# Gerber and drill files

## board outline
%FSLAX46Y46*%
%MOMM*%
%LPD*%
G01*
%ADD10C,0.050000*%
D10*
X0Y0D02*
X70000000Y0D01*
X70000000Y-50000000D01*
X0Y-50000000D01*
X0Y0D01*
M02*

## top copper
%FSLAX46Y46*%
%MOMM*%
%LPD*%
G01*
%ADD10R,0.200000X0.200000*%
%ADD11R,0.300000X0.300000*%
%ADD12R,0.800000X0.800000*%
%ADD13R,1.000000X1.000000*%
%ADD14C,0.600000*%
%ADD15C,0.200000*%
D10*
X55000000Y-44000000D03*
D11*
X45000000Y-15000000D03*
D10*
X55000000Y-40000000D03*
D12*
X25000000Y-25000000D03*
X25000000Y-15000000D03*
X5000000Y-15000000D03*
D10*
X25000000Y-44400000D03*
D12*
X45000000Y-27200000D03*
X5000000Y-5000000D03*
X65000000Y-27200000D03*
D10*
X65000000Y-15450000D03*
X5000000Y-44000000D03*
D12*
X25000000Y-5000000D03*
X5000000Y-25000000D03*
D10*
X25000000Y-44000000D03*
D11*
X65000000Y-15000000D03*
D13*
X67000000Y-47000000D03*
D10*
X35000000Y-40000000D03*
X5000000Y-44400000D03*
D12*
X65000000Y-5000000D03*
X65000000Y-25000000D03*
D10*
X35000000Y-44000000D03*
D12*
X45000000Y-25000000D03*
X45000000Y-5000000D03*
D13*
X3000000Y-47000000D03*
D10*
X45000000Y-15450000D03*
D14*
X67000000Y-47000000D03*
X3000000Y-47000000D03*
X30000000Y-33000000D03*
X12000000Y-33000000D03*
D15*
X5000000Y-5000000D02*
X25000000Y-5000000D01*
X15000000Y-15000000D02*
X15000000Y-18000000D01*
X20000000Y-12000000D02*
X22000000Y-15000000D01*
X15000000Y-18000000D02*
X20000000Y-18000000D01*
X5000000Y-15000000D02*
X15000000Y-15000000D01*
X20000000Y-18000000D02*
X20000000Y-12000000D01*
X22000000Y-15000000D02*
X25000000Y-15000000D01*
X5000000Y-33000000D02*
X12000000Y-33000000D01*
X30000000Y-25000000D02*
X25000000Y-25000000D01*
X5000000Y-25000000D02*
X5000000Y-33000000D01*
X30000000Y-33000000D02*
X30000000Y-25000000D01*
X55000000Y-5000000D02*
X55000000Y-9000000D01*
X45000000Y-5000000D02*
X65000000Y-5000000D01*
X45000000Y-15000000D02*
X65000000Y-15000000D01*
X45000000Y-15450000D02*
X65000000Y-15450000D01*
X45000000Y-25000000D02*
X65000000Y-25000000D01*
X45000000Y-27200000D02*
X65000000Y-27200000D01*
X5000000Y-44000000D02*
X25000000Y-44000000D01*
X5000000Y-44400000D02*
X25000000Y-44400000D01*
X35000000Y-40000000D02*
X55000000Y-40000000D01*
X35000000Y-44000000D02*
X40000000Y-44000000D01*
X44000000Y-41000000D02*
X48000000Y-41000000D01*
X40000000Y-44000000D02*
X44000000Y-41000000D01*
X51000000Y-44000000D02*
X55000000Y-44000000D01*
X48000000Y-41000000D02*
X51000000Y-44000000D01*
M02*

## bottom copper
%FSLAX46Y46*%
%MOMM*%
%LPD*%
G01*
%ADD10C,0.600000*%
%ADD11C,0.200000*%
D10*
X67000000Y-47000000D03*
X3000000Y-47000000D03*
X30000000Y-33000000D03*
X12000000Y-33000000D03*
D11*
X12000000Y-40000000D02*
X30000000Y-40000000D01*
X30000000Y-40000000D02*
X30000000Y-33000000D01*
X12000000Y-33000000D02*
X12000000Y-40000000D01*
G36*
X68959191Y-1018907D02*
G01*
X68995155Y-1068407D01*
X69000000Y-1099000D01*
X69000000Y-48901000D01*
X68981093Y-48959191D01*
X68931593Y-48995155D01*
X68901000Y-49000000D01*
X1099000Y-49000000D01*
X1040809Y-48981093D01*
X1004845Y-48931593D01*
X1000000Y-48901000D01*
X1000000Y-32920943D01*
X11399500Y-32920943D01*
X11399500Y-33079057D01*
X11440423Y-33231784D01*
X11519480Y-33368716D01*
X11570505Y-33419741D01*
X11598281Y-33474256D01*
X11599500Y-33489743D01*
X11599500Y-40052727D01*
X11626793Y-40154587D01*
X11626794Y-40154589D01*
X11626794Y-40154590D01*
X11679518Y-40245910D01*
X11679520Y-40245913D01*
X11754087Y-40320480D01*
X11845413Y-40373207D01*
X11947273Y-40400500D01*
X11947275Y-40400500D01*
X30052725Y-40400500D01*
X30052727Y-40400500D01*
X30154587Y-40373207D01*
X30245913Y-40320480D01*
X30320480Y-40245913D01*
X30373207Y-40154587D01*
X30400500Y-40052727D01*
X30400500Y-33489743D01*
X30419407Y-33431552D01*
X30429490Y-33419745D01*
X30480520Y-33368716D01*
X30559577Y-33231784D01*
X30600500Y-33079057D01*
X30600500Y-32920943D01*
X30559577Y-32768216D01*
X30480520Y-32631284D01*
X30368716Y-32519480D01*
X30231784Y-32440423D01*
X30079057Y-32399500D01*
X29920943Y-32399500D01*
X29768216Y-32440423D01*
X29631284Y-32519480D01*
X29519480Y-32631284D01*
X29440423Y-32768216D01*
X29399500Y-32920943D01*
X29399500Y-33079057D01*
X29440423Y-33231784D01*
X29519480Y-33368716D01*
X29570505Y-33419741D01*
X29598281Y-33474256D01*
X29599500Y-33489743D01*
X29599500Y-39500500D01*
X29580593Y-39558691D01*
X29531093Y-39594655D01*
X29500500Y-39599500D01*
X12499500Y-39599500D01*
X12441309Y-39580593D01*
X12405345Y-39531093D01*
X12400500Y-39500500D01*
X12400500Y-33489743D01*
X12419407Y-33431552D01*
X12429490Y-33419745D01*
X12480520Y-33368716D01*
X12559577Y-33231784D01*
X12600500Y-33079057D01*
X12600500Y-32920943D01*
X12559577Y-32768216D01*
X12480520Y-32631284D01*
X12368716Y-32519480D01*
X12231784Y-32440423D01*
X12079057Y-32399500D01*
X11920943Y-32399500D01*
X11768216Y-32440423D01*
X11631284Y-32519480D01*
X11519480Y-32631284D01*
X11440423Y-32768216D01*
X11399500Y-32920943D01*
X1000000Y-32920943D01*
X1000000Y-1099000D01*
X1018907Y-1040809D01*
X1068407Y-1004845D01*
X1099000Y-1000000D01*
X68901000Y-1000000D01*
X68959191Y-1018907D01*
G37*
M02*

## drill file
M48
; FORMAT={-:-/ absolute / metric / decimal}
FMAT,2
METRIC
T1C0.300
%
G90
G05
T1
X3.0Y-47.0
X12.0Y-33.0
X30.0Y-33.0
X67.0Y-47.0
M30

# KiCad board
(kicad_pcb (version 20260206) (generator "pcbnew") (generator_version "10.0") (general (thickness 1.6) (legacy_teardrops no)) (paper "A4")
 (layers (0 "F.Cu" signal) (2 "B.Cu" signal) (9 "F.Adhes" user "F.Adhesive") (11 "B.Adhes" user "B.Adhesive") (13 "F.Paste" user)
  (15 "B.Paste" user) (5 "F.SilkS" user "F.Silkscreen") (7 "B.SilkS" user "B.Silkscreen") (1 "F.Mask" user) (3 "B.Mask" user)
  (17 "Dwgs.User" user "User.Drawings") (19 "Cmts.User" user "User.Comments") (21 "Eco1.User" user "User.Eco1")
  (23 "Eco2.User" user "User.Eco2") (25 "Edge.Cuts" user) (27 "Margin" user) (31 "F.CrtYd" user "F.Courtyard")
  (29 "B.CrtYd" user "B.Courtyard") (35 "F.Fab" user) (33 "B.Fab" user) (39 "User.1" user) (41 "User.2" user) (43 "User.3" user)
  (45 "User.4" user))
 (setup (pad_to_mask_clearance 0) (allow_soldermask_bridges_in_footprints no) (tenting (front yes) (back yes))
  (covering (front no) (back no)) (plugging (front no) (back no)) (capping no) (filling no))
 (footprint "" (layer "F.Cu") (at 55 44)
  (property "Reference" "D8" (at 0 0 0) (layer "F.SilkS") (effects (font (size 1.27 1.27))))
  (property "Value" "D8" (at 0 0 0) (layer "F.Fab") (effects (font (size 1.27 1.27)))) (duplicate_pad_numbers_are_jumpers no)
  (pad "1" smd rect (at 0 0) (size 0.2 0.2) (layers "F.Cu" "F.Mask" "F.Paste") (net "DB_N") (thermal_bridge_angle 45)))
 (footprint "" (layer "F.Cu") (at 45 15)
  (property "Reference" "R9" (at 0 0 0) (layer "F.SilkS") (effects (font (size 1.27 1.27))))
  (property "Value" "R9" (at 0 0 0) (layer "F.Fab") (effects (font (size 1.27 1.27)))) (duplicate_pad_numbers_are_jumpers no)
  (pad "1" smd rect (at 0 0) (size 0.3 0.3) (layers "F.Cu" "F.Mask" "F.Paste") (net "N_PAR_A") (thermal_bridge_angle 45)))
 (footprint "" (layer "F.Cu") (at 55 40)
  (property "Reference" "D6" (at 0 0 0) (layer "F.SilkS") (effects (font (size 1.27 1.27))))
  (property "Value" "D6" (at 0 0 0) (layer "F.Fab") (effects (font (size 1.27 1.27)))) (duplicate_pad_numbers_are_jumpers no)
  (pad "1" smd rect (at 0 0) (size 0.2 0.2) (layers "F.Cu" "F.Mask" "F.Paste") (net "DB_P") (thermal_bridge_angle 45)))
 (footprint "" (layer "F.Cu") (at 25 25)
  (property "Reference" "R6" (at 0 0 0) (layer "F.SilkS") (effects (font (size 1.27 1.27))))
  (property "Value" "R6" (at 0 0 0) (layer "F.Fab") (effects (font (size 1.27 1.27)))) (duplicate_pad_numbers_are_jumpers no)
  (pad "1" smd rect (at 0 0) (size 0.8 0.8) (layers "F.Cu" "F.Mask" "F.Paste") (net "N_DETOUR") (thermal_bridge_angle 45)))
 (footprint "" (layer "F.Cu") (at 25 15)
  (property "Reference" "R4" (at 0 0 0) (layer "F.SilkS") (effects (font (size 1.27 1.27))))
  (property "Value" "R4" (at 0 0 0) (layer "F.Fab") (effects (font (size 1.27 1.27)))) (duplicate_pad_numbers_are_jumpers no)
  (pad "1" smd rect (at 0 0) (size 0.8 0.8) (layers "F.Cu" "F.Mask" "F.Paste") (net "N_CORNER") (thermal_bridge_angle 45)))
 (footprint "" (layer "F.Cu") (at 5 15)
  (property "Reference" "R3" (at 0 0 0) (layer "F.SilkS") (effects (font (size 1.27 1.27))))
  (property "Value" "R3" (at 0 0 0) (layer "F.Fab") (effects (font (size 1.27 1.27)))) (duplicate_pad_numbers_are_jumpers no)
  (pad "1" smd rect (at 0 0) (size 0.8 0.8) (layers "F.Cu" "F.Mask" "F.Paste") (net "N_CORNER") (thermal_bridge_angle 45)))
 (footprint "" (layer "F.Cu") (at 25 44.4)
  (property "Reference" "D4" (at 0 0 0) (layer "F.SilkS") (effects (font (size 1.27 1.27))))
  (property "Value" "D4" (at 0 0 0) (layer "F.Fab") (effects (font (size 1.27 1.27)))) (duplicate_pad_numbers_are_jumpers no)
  (pad "1" smd rect (at 0 0) (size 0.2 0.2) (layers "F.Cu" "F.Mask" "F.Paste") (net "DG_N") (thermal_bridge_angle 45)))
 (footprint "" (layer "F.Cu") (at 45 27.2)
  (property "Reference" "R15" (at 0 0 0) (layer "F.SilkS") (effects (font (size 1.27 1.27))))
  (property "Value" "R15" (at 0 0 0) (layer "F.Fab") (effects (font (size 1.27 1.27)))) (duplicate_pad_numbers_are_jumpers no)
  (pad "1" smd rect (at 0 0) (size 0.8 0.8) (layers "F.Cu" "F.Mask" "F.Paste") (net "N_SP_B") (thermal_bridge_angle 45)))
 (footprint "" (layer "F.Cu") (at 5 5)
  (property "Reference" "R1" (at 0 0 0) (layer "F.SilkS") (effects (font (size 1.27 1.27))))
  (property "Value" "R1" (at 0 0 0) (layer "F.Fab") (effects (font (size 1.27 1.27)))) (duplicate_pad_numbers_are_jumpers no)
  (pad "1" smd rect (at 0 0) (size 0.8 0.8) (layers "F.Cu" "F.Mask" "F.Paste") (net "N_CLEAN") (thermal_bridge_angle 45)))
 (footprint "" (layer "F.Cu") (at 65 27.2)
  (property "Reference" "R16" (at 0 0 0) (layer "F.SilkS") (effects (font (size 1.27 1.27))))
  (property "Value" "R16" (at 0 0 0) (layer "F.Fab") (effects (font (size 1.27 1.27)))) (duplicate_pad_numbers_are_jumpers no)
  (pad "1" smd rect (at 0 0) (size 0.8 0.8) (layers "F.Cu" "F.Mask" "F.Paste") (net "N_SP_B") (thermal_bridge_angle 45)))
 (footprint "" (layer "F.Cu") (at 65 15.45)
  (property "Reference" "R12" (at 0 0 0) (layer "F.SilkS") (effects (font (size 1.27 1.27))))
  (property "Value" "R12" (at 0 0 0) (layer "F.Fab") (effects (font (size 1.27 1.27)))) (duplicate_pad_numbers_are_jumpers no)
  (pad "1" smd rect (at 0 0) (size 0.2 0.2) (layers "F.Cu" "F.Mask" "F.Paste") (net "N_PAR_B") (thermal_bridge_angle 45)))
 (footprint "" (layer "F.Cu") (at 5 44)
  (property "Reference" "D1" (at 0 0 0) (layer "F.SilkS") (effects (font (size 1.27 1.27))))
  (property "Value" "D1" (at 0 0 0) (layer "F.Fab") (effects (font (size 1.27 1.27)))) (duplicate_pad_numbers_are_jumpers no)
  (pad "1" smd rect (at 0 0) (size 0.2 0.2) (layers "F.Cu" "F.Mask" "F.Paste") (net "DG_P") (thermal_bridge_angle 45)))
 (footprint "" (layer "F.Cu") (at 25 5)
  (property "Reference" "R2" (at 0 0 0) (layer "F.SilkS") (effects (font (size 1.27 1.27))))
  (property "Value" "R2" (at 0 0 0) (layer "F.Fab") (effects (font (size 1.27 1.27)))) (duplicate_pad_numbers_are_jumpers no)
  (pad "1" smd rect (at 0 0) (size 0.8 0.8) (layers "F.Cu" "F.Mask" "F.Paste") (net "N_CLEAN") (thermal_bridge_angle 45)))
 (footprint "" (layer "F.Cu") (at 5 25)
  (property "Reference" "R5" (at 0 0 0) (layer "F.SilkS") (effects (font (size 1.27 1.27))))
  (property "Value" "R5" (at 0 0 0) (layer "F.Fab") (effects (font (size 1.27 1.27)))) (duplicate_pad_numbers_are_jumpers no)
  (pad "1" smd rect (at 0 0) (size 0.8 0.8) (layers "F.Cu" "F.Mask" "F.Paste") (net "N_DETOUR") (thermal_bridge_angle 45)))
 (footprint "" (layer "F.Cu") (at 25 44)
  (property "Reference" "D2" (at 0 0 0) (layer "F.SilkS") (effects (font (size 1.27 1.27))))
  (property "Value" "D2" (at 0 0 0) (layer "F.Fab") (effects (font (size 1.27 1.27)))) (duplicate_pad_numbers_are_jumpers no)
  (pad "1" smd rect (at 0 0) (size 0.2 0.2) (layers "F.Cu" "F.Mask" "F.Paste") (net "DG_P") (thermal_bridge_angle 45)))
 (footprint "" (layer "F.Cu") (at 65 15)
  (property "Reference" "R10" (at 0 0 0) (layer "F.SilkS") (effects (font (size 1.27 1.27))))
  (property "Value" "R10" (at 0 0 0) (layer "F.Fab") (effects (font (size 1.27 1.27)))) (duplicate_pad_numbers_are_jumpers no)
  (pad "1" smd rect (at 0 0) (size 0.3 0.3) (layers "F.Cu" "F.Mask" "F.Paste") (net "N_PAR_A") (thermal_bridge_angle 45)))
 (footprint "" (layer "F.Cu") (at 67 47)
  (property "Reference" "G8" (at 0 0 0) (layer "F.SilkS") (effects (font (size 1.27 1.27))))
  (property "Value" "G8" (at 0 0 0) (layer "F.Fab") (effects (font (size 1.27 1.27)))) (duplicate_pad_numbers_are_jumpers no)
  (pad "1" smd rect (at 0 0) (size 1 1) (layers "F.Cu" "F.Mask" "F.Paste") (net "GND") (thermal_bridge_angle 45)))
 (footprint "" (layer "F.Cu") (at 35 40)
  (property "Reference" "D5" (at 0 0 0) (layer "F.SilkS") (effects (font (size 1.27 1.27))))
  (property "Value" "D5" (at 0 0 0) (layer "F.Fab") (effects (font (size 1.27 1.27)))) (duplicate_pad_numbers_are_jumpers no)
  (pad "1" smd rect (at 0 0) (size 0.2 0.2) (layers "F.Cu" "F.Mask" "F.Paste") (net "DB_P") (thermal_bridge_angle 45)))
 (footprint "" (layer "F.Cu") (at 5 44.4)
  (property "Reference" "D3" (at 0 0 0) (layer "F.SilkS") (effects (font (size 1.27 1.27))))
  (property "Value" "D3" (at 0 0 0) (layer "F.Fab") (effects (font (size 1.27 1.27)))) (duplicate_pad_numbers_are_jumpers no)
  (pad "1" smd rect (at 0 0) (size 0.2 0.2) (layers "F.Cu" "F.Mask" "F.Paste") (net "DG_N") (thermal_bridge_angle 45)))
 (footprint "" (layer "F.Cu") (at 65 5)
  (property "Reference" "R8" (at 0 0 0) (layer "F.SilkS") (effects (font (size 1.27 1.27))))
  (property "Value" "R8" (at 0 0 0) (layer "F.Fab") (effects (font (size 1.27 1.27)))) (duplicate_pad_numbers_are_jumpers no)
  (pad "1" smd rect (at 0 0) (size 0.8 0.8) (layers "F.Cu" "F.Mask" "F.Paste") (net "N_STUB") (thermal_bridge_angle 45)))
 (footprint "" (layer "F.Cu") (at 65 25)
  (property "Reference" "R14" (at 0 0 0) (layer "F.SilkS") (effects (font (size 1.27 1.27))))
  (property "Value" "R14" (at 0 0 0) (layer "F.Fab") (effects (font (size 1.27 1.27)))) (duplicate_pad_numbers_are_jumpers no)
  (pad "1" smd rect (at 0 0) (size 0.8 0.8) (layers "F.Cu" "F.Mask" "F.Paste") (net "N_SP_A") (thermal_bridge_angle 45)))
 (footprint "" (layer "F.Cu") (at 35 44)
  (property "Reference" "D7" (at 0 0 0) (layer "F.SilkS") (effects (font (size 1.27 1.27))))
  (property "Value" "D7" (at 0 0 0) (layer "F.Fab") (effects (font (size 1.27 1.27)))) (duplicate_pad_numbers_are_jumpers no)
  (pad "1" smd rect (at 0 0) (size 0.2 0.2) (layers "F.Cu" "F.Mask" "F.Paste") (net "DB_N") (thermal_bridge_angle 45)))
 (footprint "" (layer "F.Cu") (at 45 25)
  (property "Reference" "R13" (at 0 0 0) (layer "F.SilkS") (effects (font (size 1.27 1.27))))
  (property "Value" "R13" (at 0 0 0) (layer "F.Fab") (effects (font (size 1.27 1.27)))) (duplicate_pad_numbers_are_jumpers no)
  (pad "1" smd rect (at 0 0) (size 0.8 0.8) (layers "F.Cu" "F.Mask" "F.Paste") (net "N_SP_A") (thermal_bridge_angle 45)))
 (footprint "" (layer "F.Cu") (at 45 5)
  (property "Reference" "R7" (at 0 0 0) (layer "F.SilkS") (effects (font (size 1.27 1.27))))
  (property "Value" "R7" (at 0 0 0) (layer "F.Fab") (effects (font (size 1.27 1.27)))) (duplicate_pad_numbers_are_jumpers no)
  (pad "1" smd rect (at 0 0) (size 0.8 0.8) (layers "F.Cu" "F.Mask" "F.Paste") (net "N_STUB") (thermal_bridge_angle 45)))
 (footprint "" (layer "F.Cu") (at 3 47)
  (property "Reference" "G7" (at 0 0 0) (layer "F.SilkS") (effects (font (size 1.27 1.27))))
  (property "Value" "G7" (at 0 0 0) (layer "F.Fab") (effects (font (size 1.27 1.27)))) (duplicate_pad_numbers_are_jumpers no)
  (pad "1" smd rect (at 0 0) (size 1 1) (layers "F.Cu" "F.Mask" "F.Paste") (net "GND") (thermal_bridge_angle 45)))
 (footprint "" (layer "F.Cu") (at 45 15.45)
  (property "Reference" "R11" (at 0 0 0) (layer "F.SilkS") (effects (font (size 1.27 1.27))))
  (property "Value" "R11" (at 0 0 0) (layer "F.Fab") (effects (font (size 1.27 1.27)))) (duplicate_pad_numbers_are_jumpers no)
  (pad "1" smd rect (at 0 0) (size 0.2 0.2) (layers "F.Cu" "F.Mask" "F.Paste") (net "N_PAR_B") (thermal_bridge_angle 45)))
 (gr_rect (start 0 0) (end 70 50) (stroke (width 0.05) (type default)) (fill no) (layer "Edge.Cuts"))
 (via (at 67 47) (size 0.6) (drill 0.3) (layers "F.Cu" "B.Cu") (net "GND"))
 (via (at 3 47) (size 0.6) (drill 0.3) (layers "F.Cu" "B.Cu") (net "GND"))
 (segment (start 5 5) (end 25 5) (width 0.2) (layer "F.Cu") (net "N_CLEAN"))
 (segment (start 15 15) (end 15 18) (width 0.2) (layer "F.Cu") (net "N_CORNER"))
 (segment (start 20 12) (end 22 15) (width 0.2) (layer "F.Cu") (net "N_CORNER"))
 (segment (start 15 18) (end 20 18) (width 0.2) (layer "F.Cu") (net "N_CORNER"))
 (segment (start 5 15) (end 15 15) (width 0.2) (layer "F.Cu") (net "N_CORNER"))
 (segment (start 20 18) (end 20 12) (width 0.2) (layer "F.Cu") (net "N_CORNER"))
 (segment (start 22 15) (end 25 15) (width 0.2) (layer "F.Cu") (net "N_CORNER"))
 (segment (start 5 33) (end 12 33) (width 0.2) (layer "F.Cu") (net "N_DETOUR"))
 (segment (start 30 25) (end 25 25) (width 0.2) (layer "F.Cu") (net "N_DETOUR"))
 (segment (start 5 25) (end 5 33) (width 0.2) (layer "F.Cu") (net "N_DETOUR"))
 (segment (start 30 33) (end 30 25) (width 0.2) (layer "F.Cu") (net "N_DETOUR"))
 (via (at 30 33) (size 0.6) (drill 0.3) (layers "F.Cu" "B.Cu") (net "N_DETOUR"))
 (via (at 12 33) (size 0.6) (drill 0.3) (layers "F.Cu" "B.Cu") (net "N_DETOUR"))
 (segment (start 12 40) (end 30 40) (width 0.2) (layer "B.Cu") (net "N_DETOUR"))
 (segment (start 30 40) (end 30 33) (width 0.2) (layer "B.Cu") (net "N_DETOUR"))
 (segment (start 12 33) (end 12 40) (width 0.2) (layer "B.Cu") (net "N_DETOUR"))
 (segment (start 55 5) (end 55 9) (width 0.2) (layer "F.Cu") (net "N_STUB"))
 (segment (start 45 5) (end 65 5) (width 0.2) (layer "F.Cu") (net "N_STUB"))
 (segment (start 45 15) (end 65 15) (width 0.2) (layer "F.Cu") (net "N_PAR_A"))
 (segment (start 45 15.45) (end 65 15.45) (width 0.2) (layer "F.Cu") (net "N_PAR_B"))
 (segment (start 45 25) (end 65 25) (width 0.2) (layer "F.Cu") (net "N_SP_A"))
 (segment (start 45 27.2) (end 65 27.2) (width 0.2) (layer "F.Cu") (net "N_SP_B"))
 (segment (start 5 44) (end 25 44) (width 0.2) (layer "F.Cu") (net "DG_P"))
 (segment (start 5 44.4) (end 25 44.4) (width 0.2) (layer "F.Cu") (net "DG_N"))
 (segment (start 35 40) (end 55 40) (width 0.2) (layer "F.Cu") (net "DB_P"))
 (segment (start 35 44) (end 40 44) (width 0.2) (layer "F.Cu") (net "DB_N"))
 (segment (start 44 41) (end 48 41) (width 0.2) (layer "F.Cu") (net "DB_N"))
 (segment (start 40 44) (end 44 41) (width 0.2) (layer "F.Cu") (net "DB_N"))
 (segment (start 51 44) (end 55 44) (width 0.2) (layer "F.Cu") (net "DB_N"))
 (segment (start 48 41) (end 51 44) (width 0.2) (layer "F.Cu") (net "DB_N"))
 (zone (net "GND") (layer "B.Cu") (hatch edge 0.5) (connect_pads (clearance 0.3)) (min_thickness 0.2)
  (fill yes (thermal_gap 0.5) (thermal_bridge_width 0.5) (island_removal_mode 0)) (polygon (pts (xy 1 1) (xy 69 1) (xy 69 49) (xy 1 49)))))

